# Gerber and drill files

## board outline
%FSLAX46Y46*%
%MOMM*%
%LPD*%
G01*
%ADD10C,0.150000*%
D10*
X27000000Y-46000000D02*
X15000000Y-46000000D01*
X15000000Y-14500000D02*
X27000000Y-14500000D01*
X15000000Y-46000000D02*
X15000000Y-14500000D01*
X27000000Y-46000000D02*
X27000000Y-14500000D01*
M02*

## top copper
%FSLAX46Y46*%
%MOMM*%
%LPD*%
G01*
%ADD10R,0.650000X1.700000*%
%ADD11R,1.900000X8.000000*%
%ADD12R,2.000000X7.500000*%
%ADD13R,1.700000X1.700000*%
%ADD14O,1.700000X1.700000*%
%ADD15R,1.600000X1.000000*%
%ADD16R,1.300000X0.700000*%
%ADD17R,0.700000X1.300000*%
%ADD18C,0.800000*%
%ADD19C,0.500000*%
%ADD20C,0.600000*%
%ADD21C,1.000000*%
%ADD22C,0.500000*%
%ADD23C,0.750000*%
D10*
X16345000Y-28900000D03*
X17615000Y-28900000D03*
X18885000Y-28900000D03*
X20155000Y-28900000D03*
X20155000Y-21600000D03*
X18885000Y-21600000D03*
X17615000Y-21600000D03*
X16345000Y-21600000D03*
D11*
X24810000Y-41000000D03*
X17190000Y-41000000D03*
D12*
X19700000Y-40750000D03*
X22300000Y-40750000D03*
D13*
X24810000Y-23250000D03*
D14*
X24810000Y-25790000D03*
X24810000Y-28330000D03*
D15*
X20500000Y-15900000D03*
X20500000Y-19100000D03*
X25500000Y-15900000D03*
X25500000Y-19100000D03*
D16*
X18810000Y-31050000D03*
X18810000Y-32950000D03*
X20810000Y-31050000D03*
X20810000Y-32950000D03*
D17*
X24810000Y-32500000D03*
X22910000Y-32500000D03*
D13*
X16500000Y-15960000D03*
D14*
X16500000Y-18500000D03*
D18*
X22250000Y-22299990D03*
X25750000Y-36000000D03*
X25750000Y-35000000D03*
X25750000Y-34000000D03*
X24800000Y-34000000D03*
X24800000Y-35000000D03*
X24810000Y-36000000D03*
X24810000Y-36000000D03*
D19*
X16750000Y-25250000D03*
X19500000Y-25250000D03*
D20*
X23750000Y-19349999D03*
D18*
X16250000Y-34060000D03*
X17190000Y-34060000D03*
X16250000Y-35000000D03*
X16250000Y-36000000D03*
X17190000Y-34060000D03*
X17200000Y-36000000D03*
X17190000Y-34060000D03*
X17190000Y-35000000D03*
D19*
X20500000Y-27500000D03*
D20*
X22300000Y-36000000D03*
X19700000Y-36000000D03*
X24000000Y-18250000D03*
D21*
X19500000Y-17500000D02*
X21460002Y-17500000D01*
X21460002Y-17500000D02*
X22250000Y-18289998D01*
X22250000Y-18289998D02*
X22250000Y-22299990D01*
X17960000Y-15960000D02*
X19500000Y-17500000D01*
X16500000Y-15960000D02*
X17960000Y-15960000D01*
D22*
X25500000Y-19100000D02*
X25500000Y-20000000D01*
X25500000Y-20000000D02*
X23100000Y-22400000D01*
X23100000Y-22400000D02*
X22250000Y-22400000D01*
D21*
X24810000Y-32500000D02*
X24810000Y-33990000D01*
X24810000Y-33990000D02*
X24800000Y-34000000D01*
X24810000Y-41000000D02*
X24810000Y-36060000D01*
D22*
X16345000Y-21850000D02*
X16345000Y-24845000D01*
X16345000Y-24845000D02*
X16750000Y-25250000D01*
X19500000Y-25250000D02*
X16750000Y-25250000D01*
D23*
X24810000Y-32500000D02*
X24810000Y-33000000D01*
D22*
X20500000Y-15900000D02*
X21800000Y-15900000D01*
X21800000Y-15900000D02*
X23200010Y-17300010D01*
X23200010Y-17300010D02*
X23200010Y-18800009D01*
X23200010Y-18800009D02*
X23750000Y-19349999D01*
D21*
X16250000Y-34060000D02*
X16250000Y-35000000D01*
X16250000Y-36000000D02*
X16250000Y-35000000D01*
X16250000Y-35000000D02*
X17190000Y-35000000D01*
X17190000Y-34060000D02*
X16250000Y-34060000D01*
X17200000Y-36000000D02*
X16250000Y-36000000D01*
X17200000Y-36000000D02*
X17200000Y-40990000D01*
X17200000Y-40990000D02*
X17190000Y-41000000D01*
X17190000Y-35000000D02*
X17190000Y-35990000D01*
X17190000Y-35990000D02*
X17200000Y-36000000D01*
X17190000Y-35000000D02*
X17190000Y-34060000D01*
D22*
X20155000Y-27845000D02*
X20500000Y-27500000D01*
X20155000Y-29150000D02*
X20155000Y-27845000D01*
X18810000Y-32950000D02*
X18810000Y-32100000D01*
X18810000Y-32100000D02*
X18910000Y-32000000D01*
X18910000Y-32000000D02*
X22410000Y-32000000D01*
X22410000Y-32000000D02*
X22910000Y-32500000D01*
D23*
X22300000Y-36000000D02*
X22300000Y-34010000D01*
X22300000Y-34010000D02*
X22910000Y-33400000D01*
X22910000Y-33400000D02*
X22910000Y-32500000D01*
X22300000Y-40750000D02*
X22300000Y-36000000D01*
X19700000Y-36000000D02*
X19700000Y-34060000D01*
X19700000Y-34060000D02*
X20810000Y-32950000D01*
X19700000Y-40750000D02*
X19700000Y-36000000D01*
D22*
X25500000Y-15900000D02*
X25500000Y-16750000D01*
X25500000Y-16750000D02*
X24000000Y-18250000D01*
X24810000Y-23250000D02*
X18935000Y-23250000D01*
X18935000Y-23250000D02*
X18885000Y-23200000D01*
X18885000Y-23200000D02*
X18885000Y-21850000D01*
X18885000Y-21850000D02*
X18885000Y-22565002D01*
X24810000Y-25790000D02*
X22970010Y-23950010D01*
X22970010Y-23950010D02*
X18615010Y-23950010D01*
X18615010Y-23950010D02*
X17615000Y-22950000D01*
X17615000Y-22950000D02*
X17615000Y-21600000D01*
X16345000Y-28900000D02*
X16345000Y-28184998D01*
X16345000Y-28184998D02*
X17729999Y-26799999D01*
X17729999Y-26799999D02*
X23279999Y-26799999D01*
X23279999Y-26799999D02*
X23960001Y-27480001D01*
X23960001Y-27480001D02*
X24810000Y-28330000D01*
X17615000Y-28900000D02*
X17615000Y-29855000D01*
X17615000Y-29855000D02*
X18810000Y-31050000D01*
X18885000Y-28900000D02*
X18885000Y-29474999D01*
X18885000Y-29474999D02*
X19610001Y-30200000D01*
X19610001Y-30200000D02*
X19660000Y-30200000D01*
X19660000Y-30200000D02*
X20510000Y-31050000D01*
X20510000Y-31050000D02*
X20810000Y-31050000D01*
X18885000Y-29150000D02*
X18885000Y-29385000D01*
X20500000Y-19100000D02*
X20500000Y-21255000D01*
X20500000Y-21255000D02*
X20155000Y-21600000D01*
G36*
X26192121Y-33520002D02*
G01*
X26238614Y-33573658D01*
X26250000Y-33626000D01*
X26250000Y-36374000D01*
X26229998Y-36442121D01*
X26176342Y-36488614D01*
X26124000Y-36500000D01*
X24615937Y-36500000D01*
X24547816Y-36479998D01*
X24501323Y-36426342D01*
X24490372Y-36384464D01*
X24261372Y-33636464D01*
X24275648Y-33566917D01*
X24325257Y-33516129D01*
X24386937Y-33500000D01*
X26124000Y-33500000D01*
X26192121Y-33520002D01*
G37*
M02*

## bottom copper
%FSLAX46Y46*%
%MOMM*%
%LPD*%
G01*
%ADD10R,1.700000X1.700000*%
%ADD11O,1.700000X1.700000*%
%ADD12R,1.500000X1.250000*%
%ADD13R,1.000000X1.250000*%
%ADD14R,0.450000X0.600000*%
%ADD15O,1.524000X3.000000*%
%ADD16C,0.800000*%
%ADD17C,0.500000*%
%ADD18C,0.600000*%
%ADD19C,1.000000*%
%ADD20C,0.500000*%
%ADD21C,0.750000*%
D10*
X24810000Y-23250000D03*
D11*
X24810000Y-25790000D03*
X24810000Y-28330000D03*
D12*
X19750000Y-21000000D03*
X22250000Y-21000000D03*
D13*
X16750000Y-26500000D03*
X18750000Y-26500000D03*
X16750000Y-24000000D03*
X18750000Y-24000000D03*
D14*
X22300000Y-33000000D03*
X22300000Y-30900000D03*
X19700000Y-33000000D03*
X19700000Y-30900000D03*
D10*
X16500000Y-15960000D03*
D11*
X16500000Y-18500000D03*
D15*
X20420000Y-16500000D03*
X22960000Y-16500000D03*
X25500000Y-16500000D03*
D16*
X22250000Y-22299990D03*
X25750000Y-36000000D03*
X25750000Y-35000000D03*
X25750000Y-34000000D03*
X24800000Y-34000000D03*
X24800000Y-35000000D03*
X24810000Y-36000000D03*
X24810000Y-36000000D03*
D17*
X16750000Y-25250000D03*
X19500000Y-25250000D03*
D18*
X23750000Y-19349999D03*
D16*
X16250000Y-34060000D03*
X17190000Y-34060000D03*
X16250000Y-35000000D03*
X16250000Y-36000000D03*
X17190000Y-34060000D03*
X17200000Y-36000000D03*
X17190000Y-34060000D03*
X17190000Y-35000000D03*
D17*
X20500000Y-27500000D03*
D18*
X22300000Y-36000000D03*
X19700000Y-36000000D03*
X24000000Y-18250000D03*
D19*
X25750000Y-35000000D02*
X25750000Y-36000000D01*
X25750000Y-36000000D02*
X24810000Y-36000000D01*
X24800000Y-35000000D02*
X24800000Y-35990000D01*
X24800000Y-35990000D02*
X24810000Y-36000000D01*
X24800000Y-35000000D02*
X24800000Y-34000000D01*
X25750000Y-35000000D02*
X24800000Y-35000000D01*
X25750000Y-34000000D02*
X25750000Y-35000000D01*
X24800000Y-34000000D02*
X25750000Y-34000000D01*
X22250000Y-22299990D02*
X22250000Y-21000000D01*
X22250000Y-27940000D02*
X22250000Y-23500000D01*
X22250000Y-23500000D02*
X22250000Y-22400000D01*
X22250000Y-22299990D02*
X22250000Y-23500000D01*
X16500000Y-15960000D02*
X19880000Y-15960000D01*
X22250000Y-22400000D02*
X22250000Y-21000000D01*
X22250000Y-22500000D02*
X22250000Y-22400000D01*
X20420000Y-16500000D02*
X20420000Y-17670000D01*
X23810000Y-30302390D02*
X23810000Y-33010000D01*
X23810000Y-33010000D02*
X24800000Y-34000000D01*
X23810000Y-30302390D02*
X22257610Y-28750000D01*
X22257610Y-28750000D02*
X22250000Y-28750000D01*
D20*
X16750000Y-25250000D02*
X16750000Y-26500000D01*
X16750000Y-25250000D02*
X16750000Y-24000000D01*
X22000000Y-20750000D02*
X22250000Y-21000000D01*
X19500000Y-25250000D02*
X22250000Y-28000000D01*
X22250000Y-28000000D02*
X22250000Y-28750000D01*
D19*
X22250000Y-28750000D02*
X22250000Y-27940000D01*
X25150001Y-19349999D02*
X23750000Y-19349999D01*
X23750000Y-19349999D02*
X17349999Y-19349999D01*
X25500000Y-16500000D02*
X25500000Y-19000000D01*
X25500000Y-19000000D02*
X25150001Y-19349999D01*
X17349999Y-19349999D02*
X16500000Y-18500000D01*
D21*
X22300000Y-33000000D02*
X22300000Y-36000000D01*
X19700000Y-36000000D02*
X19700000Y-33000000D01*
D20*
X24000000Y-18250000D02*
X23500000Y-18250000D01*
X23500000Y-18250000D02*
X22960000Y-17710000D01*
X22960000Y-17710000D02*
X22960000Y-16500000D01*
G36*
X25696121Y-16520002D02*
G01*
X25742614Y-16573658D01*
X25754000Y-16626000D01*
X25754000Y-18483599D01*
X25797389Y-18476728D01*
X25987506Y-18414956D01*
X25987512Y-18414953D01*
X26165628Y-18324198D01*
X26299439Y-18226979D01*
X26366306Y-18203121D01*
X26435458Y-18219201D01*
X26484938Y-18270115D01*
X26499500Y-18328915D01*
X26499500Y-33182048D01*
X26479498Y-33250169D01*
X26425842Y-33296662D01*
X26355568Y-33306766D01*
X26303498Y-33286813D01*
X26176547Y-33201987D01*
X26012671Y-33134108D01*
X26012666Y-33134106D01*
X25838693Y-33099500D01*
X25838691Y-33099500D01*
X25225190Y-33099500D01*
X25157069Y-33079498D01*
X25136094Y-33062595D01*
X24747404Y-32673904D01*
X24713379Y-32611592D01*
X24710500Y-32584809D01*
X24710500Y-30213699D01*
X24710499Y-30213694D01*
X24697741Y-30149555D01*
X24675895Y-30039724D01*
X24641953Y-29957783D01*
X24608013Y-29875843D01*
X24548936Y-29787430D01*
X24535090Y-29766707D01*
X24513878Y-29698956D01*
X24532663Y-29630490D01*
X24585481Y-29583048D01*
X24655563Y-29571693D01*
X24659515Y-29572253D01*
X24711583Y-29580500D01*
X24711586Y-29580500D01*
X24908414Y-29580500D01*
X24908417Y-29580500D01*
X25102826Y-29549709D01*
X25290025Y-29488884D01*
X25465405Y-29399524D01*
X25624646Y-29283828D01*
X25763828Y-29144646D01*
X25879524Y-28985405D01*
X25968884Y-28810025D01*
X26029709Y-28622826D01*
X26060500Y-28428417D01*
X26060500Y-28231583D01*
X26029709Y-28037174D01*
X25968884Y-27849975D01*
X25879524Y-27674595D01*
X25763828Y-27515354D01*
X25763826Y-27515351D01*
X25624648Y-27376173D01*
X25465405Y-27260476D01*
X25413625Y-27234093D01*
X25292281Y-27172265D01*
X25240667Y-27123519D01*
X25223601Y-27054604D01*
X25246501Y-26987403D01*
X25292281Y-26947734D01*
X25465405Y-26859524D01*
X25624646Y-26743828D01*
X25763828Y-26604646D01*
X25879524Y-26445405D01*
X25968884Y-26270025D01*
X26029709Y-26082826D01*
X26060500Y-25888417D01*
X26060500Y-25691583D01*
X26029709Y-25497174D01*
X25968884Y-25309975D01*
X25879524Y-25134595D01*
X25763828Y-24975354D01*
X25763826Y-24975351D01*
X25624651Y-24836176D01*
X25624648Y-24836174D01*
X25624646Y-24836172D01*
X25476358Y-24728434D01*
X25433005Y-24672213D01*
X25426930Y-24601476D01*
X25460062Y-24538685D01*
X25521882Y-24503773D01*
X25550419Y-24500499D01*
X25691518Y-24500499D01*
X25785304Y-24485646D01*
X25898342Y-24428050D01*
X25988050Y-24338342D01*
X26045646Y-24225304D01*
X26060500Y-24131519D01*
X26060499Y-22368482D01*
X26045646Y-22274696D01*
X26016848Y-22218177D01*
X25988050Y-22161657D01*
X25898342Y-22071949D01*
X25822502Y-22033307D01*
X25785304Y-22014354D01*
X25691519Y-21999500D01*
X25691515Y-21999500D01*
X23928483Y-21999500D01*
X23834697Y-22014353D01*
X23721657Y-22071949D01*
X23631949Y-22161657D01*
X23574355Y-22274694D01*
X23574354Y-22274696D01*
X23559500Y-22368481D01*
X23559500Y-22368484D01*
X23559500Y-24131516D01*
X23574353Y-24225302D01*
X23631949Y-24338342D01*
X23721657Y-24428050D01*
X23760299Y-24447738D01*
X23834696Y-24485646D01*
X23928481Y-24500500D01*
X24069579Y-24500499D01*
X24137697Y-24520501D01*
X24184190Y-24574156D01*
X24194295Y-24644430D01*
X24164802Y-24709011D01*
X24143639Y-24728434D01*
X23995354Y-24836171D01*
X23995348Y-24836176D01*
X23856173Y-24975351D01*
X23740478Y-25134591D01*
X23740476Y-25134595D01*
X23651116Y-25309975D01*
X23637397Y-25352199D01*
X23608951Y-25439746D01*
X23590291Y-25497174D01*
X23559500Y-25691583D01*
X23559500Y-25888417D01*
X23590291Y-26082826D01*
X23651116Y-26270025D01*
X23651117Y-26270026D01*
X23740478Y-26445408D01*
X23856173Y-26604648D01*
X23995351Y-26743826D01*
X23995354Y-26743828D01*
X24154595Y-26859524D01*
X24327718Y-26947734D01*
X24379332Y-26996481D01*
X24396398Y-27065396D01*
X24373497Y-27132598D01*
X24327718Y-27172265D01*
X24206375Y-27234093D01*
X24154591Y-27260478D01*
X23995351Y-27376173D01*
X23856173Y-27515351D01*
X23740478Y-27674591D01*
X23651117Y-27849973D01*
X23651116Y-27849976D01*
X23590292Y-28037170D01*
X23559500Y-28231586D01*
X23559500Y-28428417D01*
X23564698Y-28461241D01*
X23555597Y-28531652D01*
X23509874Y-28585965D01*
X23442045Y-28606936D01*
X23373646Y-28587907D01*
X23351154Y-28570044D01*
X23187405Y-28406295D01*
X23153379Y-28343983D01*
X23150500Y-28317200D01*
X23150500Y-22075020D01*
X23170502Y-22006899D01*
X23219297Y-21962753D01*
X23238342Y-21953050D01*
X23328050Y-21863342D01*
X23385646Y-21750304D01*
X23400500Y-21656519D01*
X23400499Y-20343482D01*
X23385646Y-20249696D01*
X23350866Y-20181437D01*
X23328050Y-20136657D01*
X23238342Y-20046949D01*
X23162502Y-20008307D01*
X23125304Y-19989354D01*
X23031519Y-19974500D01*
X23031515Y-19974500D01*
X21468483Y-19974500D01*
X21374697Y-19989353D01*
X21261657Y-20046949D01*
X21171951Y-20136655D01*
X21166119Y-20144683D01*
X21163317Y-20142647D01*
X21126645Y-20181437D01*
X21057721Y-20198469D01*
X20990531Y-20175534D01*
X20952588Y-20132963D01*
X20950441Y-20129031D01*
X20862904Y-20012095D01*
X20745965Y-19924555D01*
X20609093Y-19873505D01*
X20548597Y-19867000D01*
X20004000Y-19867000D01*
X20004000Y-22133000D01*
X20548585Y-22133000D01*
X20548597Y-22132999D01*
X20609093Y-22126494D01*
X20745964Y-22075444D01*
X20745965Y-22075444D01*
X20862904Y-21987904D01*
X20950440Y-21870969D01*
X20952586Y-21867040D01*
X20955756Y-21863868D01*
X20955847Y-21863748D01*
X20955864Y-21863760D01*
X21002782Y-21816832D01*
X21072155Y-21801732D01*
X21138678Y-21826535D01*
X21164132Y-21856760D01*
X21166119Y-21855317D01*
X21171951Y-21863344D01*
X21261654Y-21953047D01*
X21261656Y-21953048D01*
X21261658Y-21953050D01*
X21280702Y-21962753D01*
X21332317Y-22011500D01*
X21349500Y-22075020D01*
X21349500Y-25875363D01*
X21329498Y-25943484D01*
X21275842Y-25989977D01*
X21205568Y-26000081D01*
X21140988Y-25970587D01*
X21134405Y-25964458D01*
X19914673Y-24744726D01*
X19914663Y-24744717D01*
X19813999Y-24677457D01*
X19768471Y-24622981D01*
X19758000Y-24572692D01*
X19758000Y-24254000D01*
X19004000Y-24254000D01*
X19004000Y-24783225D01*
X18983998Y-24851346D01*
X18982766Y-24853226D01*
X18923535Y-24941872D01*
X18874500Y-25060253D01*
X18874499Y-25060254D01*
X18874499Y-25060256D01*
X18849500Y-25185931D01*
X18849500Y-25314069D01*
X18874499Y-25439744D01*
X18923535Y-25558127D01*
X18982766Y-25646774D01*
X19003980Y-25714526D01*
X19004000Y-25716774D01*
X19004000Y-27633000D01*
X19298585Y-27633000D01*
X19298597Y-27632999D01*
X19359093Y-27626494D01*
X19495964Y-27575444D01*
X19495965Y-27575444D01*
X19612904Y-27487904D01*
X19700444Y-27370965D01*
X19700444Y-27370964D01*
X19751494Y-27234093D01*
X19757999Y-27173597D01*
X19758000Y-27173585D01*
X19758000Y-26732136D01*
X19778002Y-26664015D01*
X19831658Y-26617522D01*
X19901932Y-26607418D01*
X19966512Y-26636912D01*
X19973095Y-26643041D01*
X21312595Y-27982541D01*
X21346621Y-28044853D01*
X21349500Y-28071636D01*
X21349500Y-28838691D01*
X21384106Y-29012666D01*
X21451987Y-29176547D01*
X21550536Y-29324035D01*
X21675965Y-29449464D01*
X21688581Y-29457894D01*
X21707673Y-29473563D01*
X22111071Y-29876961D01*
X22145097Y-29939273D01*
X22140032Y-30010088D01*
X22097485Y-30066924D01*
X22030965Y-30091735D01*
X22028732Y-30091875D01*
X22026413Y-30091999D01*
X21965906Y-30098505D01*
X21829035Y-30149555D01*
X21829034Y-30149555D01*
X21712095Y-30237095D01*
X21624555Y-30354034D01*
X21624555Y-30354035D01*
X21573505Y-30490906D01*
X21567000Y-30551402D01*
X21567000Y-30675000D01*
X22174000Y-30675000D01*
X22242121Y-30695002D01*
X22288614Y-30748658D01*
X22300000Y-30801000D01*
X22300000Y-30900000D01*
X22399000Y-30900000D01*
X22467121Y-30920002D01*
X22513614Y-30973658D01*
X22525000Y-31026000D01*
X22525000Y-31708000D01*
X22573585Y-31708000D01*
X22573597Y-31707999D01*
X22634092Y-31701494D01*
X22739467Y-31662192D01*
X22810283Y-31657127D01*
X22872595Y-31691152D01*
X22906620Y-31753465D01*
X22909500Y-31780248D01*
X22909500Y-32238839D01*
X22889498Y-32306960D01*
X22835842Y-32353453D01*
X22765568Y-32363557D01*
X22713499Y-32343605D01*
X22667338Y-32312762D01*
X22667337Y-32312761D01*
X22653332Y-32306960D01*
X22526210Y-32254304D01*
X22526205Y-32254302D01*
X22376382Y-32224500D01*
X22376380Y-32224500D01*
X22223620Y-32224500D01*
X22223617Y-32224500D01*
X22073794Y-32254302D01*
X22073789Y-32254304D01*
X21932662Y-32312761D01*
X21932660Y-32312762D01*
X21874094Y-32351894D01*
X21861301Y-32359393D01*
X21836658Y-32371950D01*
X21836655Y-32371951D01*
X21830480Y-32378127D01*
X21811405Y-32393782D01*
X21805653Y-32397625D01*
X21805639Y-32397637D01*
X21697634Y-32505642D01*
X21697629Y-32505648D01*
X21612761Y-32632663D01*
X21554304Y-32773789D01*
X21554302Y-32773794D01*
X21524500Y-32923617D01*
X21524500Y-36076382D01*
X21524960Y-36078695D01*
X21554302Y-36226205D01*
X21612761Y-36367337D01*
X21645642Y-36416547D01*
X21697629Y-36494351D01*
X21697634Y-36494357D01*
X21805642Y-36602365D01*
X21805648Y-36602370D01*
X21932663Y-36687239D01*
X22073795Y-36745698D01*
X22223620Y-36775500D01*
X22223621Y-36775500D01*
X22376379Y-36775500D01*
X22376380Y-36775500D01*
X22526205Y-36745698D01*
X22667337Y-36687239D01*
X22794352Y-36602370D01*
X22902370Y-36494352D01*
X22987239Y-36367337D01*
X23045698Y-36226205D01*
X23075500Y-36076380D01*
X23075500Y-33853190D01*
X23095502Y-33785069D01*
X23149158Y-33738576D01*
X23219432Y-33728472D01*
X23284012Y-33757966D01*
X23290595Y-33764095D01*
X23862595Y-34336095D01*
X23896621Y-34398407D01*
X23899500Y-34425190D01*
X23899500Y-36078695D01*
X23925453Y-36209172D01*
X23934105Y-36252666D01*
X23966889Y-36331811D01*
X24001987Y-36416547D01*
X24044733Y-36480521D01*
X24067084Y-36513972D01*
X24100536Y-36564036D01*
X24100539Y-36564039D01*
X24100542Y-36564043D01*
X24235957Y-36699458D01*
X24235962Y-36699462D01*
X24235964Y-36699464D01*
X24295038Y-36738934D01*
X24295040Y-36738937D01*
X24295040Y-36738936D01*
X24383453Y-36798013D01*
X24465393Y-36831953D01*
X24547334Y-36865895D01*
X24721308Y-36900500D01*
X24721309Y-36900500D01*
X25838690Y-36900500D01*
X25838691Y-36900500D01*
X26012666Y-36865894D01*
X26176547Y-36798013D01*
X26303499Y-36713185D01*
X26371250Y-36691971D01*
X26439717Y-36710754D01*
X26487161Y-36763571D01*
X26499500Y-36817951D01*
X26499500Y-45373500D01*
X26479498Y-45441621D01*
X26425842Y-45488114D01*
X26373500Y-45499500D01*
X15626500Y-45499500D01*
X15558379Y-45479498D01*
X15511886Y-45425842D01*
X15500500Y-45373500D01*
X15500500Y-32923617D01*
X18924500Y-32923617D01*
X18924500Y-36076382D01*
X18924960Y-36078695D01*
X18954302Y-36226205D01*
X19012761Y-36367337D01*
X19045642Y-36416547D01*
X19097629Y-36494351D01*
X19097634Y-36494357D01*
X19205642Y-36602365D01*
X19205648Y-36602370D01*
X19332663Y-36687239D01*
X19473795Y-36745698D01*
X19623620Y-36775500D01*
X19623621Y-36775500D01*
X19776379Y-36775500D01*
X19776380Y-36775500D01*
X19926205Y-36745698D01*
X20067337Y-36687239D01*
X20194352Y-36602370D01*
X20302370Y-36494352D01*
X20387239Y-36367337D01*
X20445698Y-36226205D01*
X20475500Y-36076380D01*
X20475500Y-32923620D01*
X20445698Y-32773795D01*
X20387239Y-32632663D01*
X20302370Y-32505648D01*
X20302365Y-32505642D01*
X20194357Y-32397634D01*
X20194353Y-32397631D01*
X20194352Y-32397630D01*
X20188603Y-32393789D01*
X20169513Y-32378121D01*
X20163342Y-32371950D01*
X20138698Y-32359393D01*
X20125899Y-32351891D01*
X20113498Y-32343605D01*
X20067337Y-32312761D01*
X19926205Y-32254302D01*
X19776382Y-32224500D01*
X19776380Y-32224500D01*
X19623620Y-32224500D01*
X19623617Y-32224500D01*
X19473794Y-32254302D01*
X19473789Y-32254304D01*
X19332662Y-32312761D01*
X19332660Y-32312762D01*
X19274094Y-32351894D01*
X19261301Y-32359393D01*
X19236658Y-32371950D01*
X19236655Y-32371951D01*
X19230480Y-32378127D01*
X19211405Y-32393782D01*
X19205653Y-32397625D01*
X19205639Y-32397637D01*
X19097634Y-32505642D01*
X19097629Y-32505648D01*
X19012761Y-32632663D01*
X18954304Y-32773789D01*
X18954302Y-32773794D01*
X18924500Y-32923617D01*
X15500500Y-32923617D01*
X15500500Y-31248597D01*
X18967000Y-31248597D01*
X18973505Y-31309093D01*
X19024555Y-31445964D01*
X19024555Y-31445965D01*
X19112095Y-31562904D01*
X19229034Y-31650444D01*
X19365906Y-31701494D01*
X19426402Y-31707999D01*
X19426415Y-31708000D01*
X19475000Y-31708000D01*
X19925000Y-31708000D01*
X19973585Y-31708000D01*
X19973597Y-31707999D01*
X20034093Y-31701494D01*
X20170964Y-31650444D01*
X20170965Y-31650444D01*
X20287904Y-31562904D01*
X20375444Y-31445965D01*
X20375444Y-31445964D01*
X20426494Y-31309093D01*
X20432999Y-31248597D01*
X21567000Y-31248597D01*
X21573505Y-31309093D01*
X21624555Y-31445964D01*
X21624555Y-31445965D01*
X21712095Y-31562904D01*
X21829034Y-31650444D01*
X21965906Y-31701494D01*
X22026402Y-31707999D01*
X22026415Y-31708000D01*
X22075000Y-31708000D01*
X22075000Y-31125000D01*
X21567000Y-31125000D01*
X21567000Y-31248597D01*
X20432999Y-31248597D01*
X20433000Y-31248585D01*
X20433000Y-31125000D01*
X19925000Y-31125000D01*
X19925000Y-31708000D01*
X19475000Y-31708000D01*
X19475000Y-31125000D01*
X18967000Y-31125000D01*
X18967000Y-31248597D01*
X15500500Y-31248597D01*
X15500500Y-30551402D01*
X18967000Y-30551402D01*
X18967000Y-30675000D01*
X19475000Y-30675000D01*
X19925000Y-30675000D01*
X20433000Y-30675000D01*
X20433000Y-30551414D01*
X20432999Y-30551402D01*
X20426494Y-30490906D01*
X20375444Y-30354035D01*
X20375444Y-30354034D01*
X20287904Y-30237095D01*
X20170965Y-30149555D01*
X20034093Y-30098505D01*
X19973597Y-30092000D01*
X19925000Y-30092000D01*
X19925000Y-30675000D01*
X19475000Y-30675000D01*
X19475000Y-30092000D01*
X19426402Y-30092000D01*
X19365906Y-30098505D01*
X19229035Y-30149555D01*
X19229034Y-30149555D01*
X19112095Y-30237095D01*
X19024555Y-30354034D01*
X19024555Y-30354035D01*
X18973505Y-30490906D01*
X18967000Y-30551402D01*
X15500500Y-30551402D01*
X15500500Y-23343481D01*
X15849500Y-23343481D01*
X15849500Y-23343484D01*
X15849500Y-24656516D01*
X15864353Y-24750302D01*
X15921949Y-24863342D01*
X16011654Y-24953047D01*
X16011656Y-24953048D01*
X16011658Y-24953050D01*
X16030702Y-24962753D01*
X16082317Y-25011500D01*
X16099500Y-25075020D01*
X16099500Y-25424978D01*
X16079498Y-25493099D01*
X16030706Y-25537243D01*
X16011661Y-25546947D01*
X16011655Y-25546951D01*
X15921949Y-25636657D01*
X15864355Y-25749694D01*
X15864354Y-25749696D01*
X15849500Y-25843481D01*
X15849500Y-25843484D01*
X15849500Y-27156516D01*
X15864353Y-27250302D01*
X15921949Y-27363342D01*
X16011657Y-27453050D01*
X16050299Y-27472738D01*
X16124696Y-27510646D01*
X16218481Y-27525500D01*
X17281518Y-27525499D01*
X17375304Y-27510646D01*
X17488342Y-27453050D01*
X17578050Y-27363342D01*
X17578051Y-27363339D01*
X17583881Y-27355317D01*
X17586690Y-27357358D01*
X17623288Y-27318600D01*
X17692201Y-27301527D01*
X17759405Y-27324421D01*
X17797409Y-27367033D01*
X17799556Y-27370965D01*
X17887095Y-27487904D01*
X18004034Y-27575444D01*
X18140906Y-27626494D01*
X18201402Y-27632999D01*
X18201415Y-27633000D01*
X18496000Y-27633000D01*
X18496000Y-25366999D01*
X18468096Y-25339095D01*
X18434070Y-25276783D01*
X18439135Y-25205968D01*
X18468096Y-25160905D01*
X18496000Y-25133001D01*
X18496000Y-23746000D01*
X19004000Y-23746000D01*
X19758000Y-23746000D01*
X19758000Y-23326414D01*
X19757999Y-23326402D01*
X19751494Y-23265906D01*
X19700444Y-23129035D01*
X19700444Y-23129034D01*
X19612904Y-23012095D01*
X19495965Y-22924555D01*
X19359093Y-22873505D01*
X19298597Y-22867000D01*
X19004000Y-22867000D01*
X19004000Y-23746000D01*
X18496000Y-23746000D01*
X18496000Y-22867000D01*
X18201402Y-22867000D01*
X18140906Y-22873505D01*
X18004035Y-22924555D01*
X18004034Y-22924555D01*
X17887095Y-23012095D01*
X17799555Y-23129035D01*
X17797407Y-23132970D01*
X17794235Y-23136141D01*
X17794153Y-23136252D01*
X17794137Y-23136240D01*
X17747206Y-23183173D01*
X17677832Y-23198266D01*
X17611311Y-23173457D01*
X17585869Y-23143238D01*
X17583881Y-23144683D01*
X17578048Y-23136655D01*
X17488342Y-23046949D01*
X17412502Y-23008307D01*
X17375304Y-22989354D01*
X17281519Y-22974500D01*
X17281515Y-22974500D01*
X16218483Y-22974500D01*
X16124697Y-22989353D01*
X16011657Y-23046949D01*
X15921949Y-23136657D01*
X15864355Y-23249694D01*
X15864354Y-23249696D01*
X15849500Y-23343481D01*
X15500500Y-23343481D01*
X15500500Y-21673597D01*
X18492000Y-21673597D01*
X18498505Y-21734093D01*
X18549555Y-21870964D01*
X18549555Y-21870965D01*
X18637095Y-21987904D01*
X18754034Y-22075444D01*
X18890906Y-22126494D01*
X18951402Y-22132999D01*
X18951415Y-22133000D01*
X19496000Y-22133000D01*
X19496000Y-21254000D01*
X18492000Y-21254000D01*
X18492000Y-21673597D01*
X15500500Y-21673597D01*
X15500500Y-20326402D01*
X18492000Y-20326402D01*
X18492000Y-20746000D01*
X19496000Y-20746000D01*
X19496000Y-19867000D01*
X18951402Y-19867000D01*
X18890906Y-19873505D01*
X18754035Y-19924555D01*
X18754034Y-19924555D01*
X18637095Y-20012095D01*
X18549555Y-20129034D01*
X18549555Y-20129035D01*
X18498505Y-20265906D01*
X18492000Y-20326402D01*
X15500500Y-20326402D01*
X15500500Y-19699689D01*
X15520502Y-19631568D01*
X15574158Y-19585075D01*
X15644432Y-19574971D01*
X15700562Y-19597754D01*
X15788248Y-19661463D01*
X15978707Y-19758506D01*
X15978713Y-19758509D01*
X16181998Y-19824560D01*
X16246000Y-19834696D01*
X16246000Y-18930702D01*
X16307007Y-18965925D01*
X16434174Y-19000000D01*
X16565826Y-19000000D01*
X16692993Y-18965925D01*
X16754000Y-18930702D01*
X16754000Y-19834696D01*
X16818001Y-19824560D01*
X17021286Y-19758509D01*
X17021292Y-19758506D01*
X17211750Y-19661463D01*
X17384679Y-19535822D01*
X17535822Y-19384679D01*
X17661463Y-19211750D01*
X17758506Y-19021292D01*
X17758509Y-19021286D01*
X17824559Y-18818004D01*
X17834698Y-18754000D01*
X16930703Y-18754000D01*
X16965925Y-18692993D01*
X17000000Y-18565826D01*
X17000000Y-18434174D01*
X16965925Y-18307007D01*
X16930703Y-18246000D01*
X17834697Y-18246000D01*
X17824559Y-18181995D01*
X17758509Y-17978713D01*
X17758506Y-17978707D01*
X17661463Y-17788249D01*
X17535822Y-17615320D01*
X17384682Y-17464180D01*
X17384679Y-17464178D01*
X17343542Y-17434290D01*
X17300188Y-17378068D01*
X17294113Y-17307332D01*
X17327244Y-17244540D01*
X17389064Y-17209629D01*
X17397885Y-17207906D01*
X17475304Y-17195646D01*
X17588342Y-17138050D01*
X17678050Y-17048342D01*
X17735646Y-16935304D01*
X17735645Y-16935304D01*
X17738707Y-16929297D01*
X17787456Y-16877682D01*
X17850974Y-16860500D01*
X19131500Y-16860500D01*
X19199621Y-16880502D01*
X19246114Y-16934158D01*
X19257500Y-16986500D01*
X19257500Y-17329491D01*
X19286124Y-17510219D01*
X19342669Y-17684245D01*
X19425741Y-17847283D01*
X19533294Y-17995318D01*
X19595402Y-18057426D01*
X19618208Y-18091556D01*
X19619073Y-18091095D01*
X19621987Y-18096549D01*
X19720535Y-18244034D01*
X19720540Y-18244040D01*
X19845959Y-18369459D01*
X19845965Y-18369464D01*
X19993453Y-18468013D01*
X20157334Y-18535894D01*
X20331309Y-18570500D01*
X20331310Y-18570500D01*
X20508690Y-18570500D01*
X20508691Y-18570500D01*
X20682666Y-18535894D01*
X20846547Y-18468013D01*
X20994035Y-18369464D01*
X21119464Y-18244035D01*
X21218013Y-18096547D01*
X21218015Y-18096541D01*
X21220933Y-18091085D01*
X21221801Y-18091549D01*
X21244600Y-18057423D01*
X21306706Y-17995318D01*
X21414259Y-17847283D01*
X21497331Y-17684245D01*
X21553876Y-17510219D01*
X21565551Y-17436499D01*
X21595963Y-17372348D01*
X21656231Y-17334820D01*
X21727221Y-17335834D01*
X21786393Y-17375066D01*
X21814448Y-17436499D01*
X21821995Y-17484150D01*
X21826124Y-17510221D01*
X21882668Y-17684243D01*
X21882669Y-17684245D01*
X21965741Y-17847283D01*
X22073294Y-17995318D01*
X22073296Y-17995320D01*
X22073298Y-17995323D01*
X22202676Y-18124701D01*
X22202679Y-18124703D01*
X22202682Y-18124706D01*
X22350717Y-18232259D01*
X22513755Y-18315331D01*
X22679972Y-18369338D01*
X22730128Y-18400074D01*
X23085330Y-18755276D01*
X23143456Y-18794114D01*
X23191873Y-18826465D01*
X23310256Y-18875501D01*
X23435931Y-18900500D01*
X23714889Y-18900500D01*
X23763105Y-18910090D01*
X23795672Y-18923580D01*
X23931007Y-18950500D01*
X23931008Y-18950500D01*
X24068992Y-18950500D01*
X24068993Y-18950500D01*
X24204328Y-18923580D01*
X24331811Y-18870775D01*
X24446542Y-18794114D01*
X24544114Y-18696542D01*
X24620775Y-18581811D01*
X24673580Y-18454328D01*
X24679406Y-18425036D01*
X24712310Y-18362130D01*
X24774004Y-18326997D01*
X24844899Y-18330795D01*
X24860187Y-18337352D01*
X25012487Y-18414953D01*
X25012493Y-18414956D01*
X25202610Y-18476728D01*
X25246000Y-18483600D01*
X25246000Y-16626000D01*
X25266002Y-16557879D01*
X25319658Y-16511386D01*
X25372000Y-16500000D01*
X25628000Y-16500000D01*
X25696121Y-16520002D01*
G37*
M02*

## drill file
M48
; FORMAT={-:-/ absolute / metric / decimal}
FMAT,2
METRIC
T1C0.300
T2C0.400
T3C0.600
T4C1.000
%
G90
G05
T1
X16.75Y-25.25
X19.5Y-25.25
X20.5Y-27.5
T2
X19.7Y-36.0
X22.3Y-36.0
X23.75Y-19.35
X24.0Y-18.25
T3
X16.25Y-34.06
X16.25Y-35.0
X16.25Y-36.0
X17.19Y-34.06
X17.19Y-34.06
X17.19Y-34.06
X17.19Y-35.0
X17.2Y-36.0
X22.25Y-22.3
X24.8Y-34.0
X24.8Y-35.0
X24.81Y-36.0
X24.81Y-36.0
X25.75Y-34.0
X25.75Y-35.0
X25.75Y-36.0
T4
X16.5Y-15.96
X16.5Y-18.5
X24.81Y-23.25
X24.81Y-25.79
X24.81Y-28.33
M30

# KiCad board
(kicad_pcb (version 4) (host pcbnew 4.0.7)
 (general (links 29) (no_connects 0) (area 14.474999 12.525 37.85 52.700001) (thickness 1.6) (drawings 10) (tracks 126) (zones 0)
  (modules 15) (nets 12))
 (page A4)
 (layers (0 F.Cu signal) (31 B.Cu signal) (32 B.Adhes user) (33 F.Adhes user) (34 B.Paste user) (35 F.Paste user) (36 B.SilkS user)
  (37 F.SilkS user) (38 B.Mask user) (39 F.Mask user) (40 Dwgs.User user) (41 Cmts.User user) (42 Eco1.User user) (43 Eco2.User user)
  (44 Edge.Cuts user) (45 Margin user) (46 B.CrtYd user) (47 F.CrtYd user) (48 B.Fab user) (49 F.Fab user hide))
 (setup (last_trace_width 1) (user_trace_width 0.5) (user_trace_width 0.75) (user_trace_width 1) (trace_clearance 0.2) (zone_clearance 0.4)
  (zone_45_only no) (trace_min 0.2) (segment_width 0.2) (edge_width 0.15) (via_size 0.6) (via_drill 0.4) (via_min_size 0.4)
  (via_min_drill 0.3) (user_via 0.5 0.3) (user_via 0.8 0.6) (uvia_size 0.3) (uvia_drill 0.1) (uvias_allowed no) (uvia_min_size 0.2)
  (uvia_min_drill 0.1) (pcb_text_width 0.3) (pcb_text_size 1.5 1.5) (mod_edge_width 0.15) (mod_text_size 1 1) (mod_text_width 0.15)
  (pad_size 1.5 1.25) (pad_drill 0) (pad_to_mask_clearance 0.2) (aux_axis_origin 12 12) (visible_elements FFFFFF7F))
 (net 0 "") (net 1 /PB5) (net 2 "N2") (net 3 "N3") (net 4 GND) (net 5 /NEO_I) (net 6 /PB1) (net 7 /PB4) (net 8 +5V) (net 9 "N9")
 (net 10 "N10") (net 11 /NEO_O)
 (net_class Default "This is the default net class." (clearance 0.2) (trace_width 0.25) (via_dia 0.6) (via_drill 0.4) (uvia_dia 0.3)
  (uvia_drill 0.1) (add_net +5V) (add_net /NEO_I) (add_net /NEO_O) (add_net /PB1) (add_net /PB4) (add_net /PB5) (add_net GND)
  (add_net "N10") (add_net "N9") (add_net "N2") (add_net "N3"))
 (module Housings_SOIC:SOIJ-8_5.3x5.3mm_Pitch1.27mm (layer F.Cu) (at 18.25 25.25 90)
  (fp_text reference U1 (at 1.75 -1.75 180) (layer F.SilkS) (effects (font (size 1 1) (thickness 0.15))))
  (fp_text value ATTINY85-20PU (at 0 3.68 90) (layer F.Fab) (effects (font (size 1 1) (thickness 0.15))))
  (pad 1 smd rect (at -3.65 -1.905 90) (size 1.7 0.65) (layers F.Cu F.Paste F.Mask) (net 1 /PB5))
  (pad 2 smd rect (at -3.65 -0.635 90) (size 1.7 0.65) (layers F.Cu F.Paste F.Mask) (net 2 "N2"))
  (pad 3 smd rect (at -3.65 0.635 90) (size 1.7 0.65) (layers F.Cu F.Paste F.Mask) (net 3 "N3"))
  (pad 4 smd rect (at -3.65 1.905 90) (size 1.7 0.65) (layers F.Cu F.Paste F.Mask) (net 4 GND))
  (pad 5 smd rect (at 3.65 1.905 90) (size 1.7 0.65) (layers F.Cu F.Paste F.Mask) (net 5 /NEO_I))
  (pad 6 smd rect (at 3.65 0.635 90) (size 1.7 0.65) (layers F.Cu F.Paste F.Mask) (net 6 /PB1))
  (pad 7 smd rect (at 3.65 -0.635 90) (size 1.7 0.65) (layers F.Cu F.Paste F.Mask) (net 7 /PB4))
  (pad 8 smd rect (at 3.65 -1.905 90) (size 1.7 0.65) (layers F.Cu F.Paste F.Mask) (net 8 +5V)))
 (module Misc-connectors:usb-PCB (layer F.Cu) (at 21 45.9)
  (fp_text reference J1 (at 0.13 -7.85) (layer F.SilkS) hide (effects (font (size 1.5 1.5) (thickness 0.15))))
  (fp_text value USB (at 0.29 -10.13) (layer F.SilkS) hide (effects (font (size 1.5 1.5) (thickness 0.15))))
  (pad 1 connect rect (at 3.81 -4.9) (size 1.9 8) (layers F.Cu F.Mask) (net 8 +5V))
  (pad 4 connect rect (at -3.81 -4.9) (size 1.9 8) (layers F.Cu F.Mask) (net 4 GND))
  (pad 3 connect rect (at -1.3 -5.15) (size 2 7.5) (layers F.Cu F.Mask) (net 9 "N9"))
  (pad 2 connect rect (at 1.3 -5.15) (size 2 7.5) (layers F.Cu F.Mask) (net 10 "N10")))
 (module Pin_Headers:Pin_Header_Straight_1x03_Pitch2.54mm (layer F.Cu) (at 24.81 23.25)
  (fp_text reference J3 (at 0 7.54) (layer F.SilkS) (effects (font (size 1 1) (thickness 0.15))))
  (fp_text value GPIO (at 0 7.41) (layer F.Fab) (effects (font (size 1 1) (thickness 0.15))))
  (pad 1 thru_hole rect (at 0 0) (size 1.7 1.7) (drill 1) (layers *.Cu *.Mask) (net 6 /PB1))
  (pad 2 thru_hole oval (at 0 2.54) (size 1.7 1.7) (drill 1) (layers *.Cu *.Mask) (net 7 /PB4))
  (pad 3 thru_hole oval (at 0 5.08) (size 1.7 1.7) (drill 1) (layers *.Cu *.Mask) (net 1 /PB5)))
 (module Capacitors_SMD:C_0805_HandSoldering (layer B.Cu) (at 21 21)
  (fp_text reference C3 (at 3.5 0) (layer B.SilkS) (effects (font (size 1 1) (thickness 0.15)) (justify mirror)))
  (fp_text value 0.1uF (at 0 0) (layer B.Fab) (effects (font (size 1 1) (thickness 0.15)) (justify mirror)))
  (pad 1 smd rect (at -1.25 0) (size 1.5 1.25) (layers B.Cu B.Paste B.Mask) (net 4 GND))
  (pad 2 smd rect (at 1.25 0) (size 1.5 1.25) (layers B.Cu B.Paste B.Mask) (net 8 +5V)))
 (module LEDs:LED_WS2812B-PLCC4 (layer F.Cu) (at 23 17.5 180)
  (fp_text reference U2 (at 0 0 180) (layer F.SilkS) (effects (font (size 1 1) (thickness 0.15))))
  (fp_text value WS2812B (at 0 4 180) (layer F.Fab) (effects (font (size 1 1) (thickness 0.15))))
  (pad 3 smd rect (at 2.5 1.6 180) (size 1.6 1) (layers F.Cu F.Paste F.Mask) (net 4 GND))
  (pad 4 smd rect (at 2.5 -1.6 180) (size 1.6 1) (layers F.Cu F.Paste F.Mask) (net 5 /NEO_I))
  (pad 2 smd rect (at -2.5 1.6 180) (size 1.6 1) (layers F.Cu F.Paste F.Mask) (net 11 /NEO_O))
  (pad 1 smd rect (at -2.5 -1.6 180) (size 1.6 1) (layers F.Cu F.Paste F.Mask) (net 8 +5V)))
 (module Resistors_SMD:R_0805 (layer F.Cu) (at 18.81 32 270)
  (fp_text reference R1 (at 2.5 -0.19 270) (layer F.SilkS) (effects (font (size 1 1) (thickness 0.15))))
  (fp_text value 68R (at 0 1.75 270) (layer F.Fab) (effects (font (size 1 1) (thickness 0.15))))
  (pad 1 smd rect (at -0.95 0 270) (size 0.7 1.3) (layers F.Cu F.Paste F.Mask) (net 2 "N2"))
  (pad 2 smd rect (at 0.95 0 270) (size 0.7 1.3) (layers F.Cu F.Paste F.Mask) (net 10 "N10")))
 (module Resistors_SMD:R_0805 (layer F.Cu) (at 20.81 32 270)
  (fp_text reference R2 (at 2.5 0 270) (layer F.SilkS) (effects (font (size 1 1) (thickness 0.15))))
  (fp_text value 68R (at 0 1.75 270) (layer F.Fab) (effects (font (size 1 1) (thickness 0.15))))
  (pad 1 smd rect (at -0.95 0 270) (size 0.7 1.3) (layers F.Cu F.Paste F.Mask) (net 3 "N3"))
  (pad 2 smd rect (at 0.95 0 270) (size 0.7 1.3) (layers F.Cu F.Paste F.Mask) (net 9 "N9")))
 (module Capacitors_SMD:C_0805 (layer B.Cu) (at 17.75 26.5)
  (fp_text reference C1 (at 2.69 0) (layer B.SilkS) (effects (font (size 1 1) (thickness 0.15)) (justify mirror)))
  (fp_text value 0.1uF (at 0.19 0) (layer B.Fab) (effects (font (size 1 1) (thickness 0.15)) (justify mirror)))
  (pad 1 smd rect (at -1 0) (size 1 1.25) (layers B.Cu B.Paste B.Mask) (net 8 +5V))
  (pad 2 smd rect (at 1 0) (size 1 1.25) (layers B.Cu B.Paste B.Mask) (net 4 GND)))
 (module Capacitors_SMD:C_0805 (layer B.Cu) (at 17.75 24)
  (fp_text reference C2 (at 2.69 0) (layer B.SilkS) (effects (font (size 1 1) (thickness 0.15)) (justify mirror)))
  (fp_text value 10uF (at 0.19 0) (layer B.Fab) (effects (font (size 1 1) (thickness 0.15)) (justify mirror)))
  (pad 1 smd rect (at -1 0) (size 1 1.25) (layers B.Cu B.Paste B.Mask) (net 8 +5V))
  (pad 2 smd rect (at 1 0) (size 1 1.25) (layers B.Cu B.Paste B.Mask) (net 4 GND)))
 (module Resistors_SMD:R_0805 (layer F.Cu) (at 23.86 32.5 180)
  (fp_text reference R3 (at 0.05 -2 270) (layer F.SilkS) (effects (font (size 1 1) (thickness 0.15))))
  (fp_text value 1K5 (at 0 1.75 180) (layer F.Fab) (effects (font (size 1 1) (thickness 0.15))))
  (pad 1 smd rect (at -0.95 0 180) (size 0.7 1.3) (layers F.Cu F.Paste F.Mask) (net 8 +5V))
  (pad 2 smd rect (at 0.95 0 180) (size 0.7 1.3) (layers F.Cu F.Paste F.Mask) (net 10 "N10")))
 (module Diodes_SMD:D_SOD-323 (layer B.Cu) (at 22.3 31.95 90)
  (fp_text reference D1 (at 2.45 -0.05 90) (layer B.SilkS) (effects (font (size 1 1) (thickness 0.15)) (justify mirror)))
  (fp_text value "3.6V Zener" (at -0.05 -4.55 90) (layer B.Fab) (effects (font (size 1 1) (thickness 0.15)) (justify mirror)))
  (pad 1 smd rect (at -1.05 0 90) (size 0.6 0.45) (layers B.Cu B.Paste B.Mask) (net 10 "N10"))
  (pad 2 smd rect (at 1.05 0 90) (size 0.6 0.45) (layers B.Cu B.Paste B.Mask) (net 4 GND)))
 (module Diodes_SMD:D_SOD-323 (layer B.Cu) (at 19.7 31.95 90)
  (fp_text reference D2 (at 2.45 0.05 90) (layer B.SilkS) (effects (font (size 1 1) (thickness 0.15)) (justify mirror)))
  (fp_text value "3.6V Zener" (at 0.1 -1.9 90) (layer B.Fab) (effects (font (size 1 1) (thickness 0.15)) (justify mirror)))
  (pad 1 smd rect (at -1.05 0 90) (size 0.6 0.45) (layers B.Cu B.Paste B.Mask) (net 9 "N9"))
  (pad 2 smd rect (at 1.05 0 90) (size 0.6 0.45) (layers B.Cu B.Paste B.Mask) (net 4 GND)))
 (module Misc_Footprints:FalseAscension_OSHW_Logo (layer B.Cu) (at 16.5 35 270)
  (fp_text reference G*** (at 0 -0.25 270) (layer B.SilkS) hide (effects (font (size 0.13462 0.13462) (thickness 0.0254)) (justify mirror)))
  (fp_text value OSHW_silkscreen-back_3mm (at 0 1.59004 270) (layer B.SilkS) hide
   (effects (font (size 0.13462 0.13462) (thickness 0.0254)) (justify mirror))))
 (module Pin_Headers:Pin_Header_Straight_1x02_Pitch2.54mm (layer F.Cu) (at 16.5 15.96)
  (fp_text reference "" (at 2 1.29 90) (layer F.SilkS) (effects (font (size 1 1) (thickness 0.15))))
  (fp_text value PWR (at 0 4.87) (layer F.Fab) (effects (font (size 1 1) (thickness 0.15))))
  (pad 1 thru_hole rect (at 0 0) (size 1.7 1.7) (drill 1) (layers *.Cu *.Mask) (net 8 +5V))
  (pad 2 thru_hole oval (at 0 2.54) (size 1.7 1.7) (drill 1) (layers *.Cu *.Mask) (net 4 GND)))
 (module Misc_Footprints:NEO (layer B.Cu) (at 20.42 16.5 270)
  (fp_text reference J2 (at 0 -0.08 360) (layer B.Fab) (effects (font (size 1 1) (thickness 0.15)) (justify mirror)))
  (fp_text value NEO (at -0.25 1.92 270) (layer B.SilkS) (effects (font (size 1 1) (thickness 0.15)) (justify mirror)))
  (pad 1 smd oval (at 0 0 270) (size 3 1.524) (layers B.Cu B.Paste B.Mask) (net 8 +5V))
  (pad 2 smd oval (at 0 -2.54 270) (size 3 1.524) (layers B.Cu B.Paste B.Mask) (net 11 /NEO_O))
  (pad 3 smd oval (at 0 -5.08 270) (size 3 1.524) (layers B.Cu B.Paste B.Mask) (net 4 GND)))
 (gr_line (start 27 46) (end 15 46) (layer Edge.Cuts) (width 0.15))
 (gr_line (start 15 14.5) (end 27 14.5) (layer Edge.Cuts) (width 0.15))
 (gr_line (start 15 46) (end 15 14.5) (layer Edge.Cuts) (width 0.15))
 (gr_line (start 27 46) (end 27 14.5) (layer Edge.Cuts) (width 0.15))
 (segment (start 25.75 35) (end 25.75 36) (width 1) (layer B.Cu) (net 8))
 (segment (start 25.75 36) (end 24.81 36) (width 1) (layer B.Cu) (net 8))
 (segment (start 24.8 35) (end 24.8 35.99) (width 1) (layer B.Cu) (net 8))
 (segment (start 24.8 35.99) (end 24.81 36) (width 1) (layer B.Cu) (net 8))
 (segment (start 24.8 35) (end 24.8 34) (width 1) (layer B.Cu) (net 8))
 (segment (start 25.75 35) (end 24.8 35) (width 1) (layer B.Cu) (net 8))
 (segment (start 25.75 34) (end 25.75 35) (width 1) (layer B.Cu) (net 8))
 (segment (start 24.8 34) (end 25.75 34) (width 1) (layer B.Cu) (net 8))
 (segment (start 22.25 22.29999) (end 22.25 21) (width 1) (layer B.Cu) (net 8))
 (segment (start 22.25 27.94) (end 22.25 23.5) (width 1) (layer B.Cu) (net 8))
 (segment (start 22.25 23.5) (end 22.25 22.4) (width 1) (layer B.Cu) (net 8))
 (segment (start 22.25 22.29999) (end 22.25 23.5) (width 1) (layer B.Cu) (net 8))
 (via (at 22.25 22.29999) (size 0.8) (drill 0.6) (layers F.Cu B.Cu) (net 8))
 (segment (start 19.5 17.5) (end 21.460002 17.5) (width 1) (layer F.Cu) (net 8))
 (segment (start 21.460002 17.5) (end 22.25 18.289998) (width 1) (layer F.Cu) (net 8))
 (segment (start 22.25 18.289998) (end 22.25 22.29999) (width 1) (layer F.Cu) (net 8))
 (segment (start 17.96 15.96) (end 19.5 17.5) (width 1) (layer F.Cu) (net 8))
 (segment (start 16.5 15.96) (end 17.96 15.96) (width 1) (layer F.Cu) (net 8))
 (segment (start 16.5 15.96) (end 19.88 15.96) (width 1) (layer B.Cu) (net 8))
 (segment (start 25.5 19.1) (end 25.5 20) (width 0.5) (layer F.Cu) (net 8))
 (segment (start 25.5 20) (end 23.1 22.4) (width 0.5) (layer F.Cu) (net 8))
 (segment (start 23.1 22.4) (end 22.25 22.4) (width 0.5) (layer F.Cu) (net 8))
 (segment (start 22.25 22.4) (end 22.25 21) (width 1) (layer B.Cu) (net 8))
 (segment (start 22.25 22.5) (end 22.25 22.4) (width 1) (layer B.Cu) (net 8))
 (via (at 25.75 36) (size 0.8) (drill 0.6) (layers F.Cu B.Cu) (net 8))
 (via (at 25.75 35) (size 0.8) (drill 0.6) (layers F.Cu B.Cu) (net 8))
 (via (at 25.75 34) (size 0.8) (drill 0.6) (layers F.Cu B.Cu) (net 8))
 (segment (start 20.42 16.5) (end 20.42 17.67) (width 1) (layer B.Cu) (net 8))
 (segment (start 23.81 30.30239) (end 23.81 33.01) (width 1) (layer B.Cu) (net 8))
 (segment (start 23.81 33.01) (end 24.8 34) (width 1) (layer B.Cu) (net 8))
 (segment (start 24.81 32.5) (end 24.81 33.99) (width 1) (layer F.Cu) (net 8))
 (segment (start 24.81 33.99) (end 24.8 34) (width 1) (layer F.Cu) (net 8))
 (via (at 24.8 34) (size 0.8) (drill 0.6) (layers F.Cu B.Cu) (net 8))
 (segment (start 23.81 30.30239) (end 22.25761 28.75) (width 1) (layer B.Cu) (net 8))
 (segment (start 22.25761 28.75) (end 22.25 28.75) (width 1) (layer B.Cu) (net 8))
 (via (at 24.8 35) (size 0.8) (drill 0.6) (layers F.Cu B.Cu) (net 8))
 (via (at 24.81 36) (size 0.8) (drill 0.6) (layers F.Cu B.Cu) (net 8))
 (segment (start 24.81 41) (end 24.81 36.06) (width 1) (layer F.Cu) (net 8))
 (via (at 24.81 36) (size 0.8) (drill 0.6) (layers F.Cu B.Cu) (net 8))
 (segment (start 16.345 21.85) (end 16.345 24.845) (width 0.5) (layer F.Cu) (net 8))
 (segment (start 16.345 24.845) (end 16.75 25.25) (width 0.5) (layer F.Cu) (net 8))
 (segment (start 16.75 25.25) (end 16.75 26.5) (width 0.5) (layer B.Cu) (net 8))
 (segment (start 16.75 25.25) (end 16.75 24) (width 0.5) (layer B.Cu) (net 8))
 (segment (start 19.5 25.25) (end 16.75 25.25) (width 0.5) (layer F.Cu) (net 8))
 (via (at 16.75 25.25) (size 0.5) (drill 0.3) (layers F.Cu B.Cu) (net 8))
 (via (at 19.5 25.25) (size 0.5) (drill 0.3) (layers F.Cu B.Cu) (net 8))
 (segment (start 22 20.75) (end 22.25 21) (width 0.5) (layer B.Cu) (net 8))
 (segment (start 24.81 32.5) (end 24.81 33) (width 0.75) (layer F.Cu) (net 8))
 (segment (start 19.5 25.25) (end 22.25 28) (width 0.5) (layer B.Cu) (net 8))
 (segment (start 22.25 28) (end 22.25 28.75) (width 0.5) (layer B.Cu) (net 8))
 (segment (start 22.25 28.75) (end 22.25 27.94) (width 1) (layer B.Cu) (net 8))
 (via (at 23.75 19.349999) (size 0.6) (drill 0.4) (layers F.Cu B.Cu) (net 4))
 (segment (start 25.150001 19.349999) (end 23.75 19.349999) (width 1) (layer B.Cu) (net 4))
 (segment (start 23.75 19.349999) (end 17.349999 19.349999) (width 1) (layer B.Cu) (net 4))
 (segment (start 20.5 15.9) (end 21.8 15.9) (width 0.5) (layer F.Cu) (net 4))
 (segment (start 21.8 15.9) (end 23.20001 17.30001) (width 0.5) (layer F.Cu) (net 4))
 (segment (start 23.20001 17.30001) (end 23.20001 18.800009) (width 0.5) (layer F.Cu) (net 4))
 (segment (start 23.20001 18.800009) (end 23.75 19.349999) (width 0.5) (layer F.Cu) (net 4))
 (segment (start 25.5 16.5) (end 25.5 19) (width 1) (layer B.Cu) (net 4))
 (segment (start 25.5 19) (end 25.150001 19.349999) (width 1) (layer B.Cu) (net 4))
 (segment (start 17.349999 19.349999) (end 16.5 18.5) (width 1) (layer B.Cu) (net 4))
 (segment (start 16.25 34.06) (end 16.25 35) (width 1) (layer F.Cu) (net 4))
 (segment (start 16.25 36) (end 16.25 35) (width 1) (layer F.Cu) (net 4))
 (segment (start 16.25 35) (end 17.19 35) (width 1) (layer F.Cu) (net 4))
 (segment (start 17.19 34.06) (end 16.25 34.06) (width 1) (layer F.Cu) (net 4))
 (via (at 16.25 34.06) (size 0.8) (drill 0.6) (layers F.Cu B.Cu) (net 4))
 (via (at 17.19 34.06) (size 0.8) (drill 0.6) (layers F.Cu B.Cu) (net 4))
 (via (at 16.25 35) (size 0.8) (drill 0.6) (layers F.Cu B.Cu) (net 4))
 (segment (start 17.2 36) (end 16.25 36) (width 1) (layer F.Cu) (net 4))
 (via (at 16.25 36) (size 0.8) (drill 0.6) (layers F.Cu B.Cu) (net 4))
 (via (at 17.19 34.06) (size 0.8) (drill 0.6) (layers F.Cu B.Cu) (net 4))
 (segment (start 17.2 36) (end 17.2 40.99) (width 1) (layer F.Cu) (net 4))
 (segment (start 17.2 40.99) (end 17.19 41) (width 1) (layer F.Cu) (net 4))
 (segment (start 17.19 35) (end 17.19 35.99) (width 1) (layer F.Cu) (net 4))
 (via (at 17.2 36) (size 0.8) (drill 0.6) (layers F.Cu B.Cu) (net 4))
 (segment (start 17.19 35.99) (end 17.2 36) (width 1) (layer F.Cu) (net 4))
 (via (at 17.19 34.06) (size 0.8) (drill 0.6) (layers F.Cu B.Cu) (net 4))
 (via (at 17.19 35) (size 0.8) (drill 0.6) (layers F.Cu B.Cu) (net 4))
 (segment (start 17.19 35) (end 17.19 34.06) (width 1) (layer F.Cu) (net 4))
 (via (at 20.5 27.5) (size 0.5) (drill 0.3) (layers F.Cu B.Cu) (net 4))
 (segment (start 20.155 27.845) (end 20.5 27.5) (width 0.5) (layer F.Cu) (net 4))
 (segment (start 20.155 29.15) (end 20.155 27.845) (width 0.5) (layer F.Cu) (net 4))
 (segment (start 18.81 32.95) (end 18.81 32.1) (width 0.5) (layer F.Cu) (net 10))
 (segment (start 18.81 32.1) (end 18.91 32) (width 0.5) (layer F.Cu) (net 10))
 (segment (start 18.91 32) (end 22.41 32) (width 0.5) (layer F.Cu) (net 10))
 (segment (start 22.41 32) (end 22.91 32.5) (width 0.5) (layer F.Cu) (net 10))
 (segment (start 22.3 36) (end 22.3 34.01) (width 0.75) (layer F.Cu) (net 10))
 (segment (start 22.3 34.01) (end 22.91 33.4) (width 0.75) (layer F.Cu) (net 10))
 (segment (start 22.91 33.4) (end 22.91 32.5) (width 0.75) (layer F.Cu) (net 10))
 (segment (start 22.3 33) (end 22.3 36) (width 0.75) (layer B.Cu) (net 10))
 (segment (start 22.3 40.75) (end 22.3 36) (width 0.75) (layer F.Cu) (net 10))
 (via (at 22.3 36) (size 0.6) (drill 0.4) (layers F.Cu B.Cu) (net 10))
 (segment (start 19.7 36) (end 19.7 34.06) (width 0.75) (layer F.Cu) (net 9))
 (segment (start 19.7 34.06) (end 20.81 32.95) (width 0.75) (layer F.Cu) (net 9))
 (segment (start 19.7 36) (end 19.7 33) (width 0.75) (layer B.Cu) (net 9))
 (segment (start 19.7 40.75) (end 19.7 36) (width 0.75) (layer F.Cu) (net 9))
 (via (at 19.7 36) (size 0.6) (drill 0.4) (layers F.Cu B.Cu) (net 9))
 (segment (start 24 18.25) (end 23.5 18.25) (width 0.5) (layer B.Cu) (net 11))
 (segment (start 23.5 18.25) (end 22.96 17.71) (width 0.5) (layer B.Cu) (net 11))
 (segment (start 22.96 17.71) (end 22.96 16.5) (width 0.5) (layer B.Cu) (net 11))
 (segment (start 25.5 15.9) (end 25.5 16.75) (width 0.5) (layer F.Cu) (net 11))
 (segment (start 25.5 16.75) (end 24 18.25) (width 0.5) (layer F.Cu) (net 11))
 (via (at 24 18.25) (size 0.6) (drill 0.4) (layers F.Cu B.Cu) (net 11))
 (segment (start 24.81 23.25) (end 18.935 23.25) (width 0.5) (layer F.Cu) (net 6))
 (segment (start 18.935 23.25) (end 18.885 23.2) (width 0.5) (layer F.Cu) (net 6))
 (segment (start 18.885 23.2) (end 18.885 21.85) (width 0.5) (layer F.Cu) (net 6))
 (segment (start 18.885 21.85) (end 18.885 22.565002) (width 0.5) (layer F.Cu) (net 6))
 (segment (start 24.81 25.79) (end 22.97001 23.95001) (width 0.5) (layer F.Cu) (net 7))
 (segment (start 22.97001 23.95001) (end 18.61501 23.95001) (width 0.5) (layer F.Cu) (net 7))
 (segment (start 18.61501 23.95001) (end 17.615 22.95) (width 0.5) (layer F.Cu) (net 7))
 (segment (start 17.615 22.95) (end 17.615 21.6) (width 0.5) (layer F.Cu) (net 7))
 (segment (start 16.345 28.9) (end 16.345 28.184998) (width 0.5) (layer F.Cu) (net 1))
 (segment (start 16.345 28.184998) (end 17.729999 26.799999) (width 0.5) (layer F.Cu) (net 1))
 (segment (start 17.729999 26.799999) (end 23.279999 26.799999) (width 0.5) (layer F.Cu) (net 1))
 (segment (start 23.279999 26.799999) (end 23.960001 27.480001) (width 0.5) (layer F.Cu) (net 1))
 (segment (start 23.960001 27.480001) (end 24.81 28.33) (width 0.5) (layer F.Cu) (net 1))
 (segment (start 17.615 28.9) (end 17.615 29.855) (width 0.5) (layer F.Cu) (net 2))
 (segment (start 17.615 29.855) (end 18.81 31.05) (width 0.5) (layer F.Cu) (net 2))
 (segment (start 18.885 28.9) (end 18.885 29.474999) (width 0.5) (layer F.Cu) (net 3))
 (segment (start 18.885 29.474999) (end 19.610001 30.2) (width 0.5) (layer F.Cu) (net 3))
 (segment (start 19.610001 30.2) (end 19.66 30.2) (width 0.5) (layer F.Cu) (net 3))
 (segment (start 19.66 30.2) (end 20.51 31.05) (width 0.5) (layer F.Cu) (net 3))
 (segment (start 20.51 31.05) (end 20.81 31.05) (width 0.5) (layer F.Cu) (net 3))
 (segment (start 18.885 29.15) (end 18.885 29.385) (width 0.5) (layer F.Cu) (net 3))
 (segment (start 20.5 19.1) (end 20.5 21.255) (width 0.5) (layer F.Cu) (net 5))
 (segment (start 20.5 21.255) (end 20.155 21.6) (width 0.5) (layer F.Cu) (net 5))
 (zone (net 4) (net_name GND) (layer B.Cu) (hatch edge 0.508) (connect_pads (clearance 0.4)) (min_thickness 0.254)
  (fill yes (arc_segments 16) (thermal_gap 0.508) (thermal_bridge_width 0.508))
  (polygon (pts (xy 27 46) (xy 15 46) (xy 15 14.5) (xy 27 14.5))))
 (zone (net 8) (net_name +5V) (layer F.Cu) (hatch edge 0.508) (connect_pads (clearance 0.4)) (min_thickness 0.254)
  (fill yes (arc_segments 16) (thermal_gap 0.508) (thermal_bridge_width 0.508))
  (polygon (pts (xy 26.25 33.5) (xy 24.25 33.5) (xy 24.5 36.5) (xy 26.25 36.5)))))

